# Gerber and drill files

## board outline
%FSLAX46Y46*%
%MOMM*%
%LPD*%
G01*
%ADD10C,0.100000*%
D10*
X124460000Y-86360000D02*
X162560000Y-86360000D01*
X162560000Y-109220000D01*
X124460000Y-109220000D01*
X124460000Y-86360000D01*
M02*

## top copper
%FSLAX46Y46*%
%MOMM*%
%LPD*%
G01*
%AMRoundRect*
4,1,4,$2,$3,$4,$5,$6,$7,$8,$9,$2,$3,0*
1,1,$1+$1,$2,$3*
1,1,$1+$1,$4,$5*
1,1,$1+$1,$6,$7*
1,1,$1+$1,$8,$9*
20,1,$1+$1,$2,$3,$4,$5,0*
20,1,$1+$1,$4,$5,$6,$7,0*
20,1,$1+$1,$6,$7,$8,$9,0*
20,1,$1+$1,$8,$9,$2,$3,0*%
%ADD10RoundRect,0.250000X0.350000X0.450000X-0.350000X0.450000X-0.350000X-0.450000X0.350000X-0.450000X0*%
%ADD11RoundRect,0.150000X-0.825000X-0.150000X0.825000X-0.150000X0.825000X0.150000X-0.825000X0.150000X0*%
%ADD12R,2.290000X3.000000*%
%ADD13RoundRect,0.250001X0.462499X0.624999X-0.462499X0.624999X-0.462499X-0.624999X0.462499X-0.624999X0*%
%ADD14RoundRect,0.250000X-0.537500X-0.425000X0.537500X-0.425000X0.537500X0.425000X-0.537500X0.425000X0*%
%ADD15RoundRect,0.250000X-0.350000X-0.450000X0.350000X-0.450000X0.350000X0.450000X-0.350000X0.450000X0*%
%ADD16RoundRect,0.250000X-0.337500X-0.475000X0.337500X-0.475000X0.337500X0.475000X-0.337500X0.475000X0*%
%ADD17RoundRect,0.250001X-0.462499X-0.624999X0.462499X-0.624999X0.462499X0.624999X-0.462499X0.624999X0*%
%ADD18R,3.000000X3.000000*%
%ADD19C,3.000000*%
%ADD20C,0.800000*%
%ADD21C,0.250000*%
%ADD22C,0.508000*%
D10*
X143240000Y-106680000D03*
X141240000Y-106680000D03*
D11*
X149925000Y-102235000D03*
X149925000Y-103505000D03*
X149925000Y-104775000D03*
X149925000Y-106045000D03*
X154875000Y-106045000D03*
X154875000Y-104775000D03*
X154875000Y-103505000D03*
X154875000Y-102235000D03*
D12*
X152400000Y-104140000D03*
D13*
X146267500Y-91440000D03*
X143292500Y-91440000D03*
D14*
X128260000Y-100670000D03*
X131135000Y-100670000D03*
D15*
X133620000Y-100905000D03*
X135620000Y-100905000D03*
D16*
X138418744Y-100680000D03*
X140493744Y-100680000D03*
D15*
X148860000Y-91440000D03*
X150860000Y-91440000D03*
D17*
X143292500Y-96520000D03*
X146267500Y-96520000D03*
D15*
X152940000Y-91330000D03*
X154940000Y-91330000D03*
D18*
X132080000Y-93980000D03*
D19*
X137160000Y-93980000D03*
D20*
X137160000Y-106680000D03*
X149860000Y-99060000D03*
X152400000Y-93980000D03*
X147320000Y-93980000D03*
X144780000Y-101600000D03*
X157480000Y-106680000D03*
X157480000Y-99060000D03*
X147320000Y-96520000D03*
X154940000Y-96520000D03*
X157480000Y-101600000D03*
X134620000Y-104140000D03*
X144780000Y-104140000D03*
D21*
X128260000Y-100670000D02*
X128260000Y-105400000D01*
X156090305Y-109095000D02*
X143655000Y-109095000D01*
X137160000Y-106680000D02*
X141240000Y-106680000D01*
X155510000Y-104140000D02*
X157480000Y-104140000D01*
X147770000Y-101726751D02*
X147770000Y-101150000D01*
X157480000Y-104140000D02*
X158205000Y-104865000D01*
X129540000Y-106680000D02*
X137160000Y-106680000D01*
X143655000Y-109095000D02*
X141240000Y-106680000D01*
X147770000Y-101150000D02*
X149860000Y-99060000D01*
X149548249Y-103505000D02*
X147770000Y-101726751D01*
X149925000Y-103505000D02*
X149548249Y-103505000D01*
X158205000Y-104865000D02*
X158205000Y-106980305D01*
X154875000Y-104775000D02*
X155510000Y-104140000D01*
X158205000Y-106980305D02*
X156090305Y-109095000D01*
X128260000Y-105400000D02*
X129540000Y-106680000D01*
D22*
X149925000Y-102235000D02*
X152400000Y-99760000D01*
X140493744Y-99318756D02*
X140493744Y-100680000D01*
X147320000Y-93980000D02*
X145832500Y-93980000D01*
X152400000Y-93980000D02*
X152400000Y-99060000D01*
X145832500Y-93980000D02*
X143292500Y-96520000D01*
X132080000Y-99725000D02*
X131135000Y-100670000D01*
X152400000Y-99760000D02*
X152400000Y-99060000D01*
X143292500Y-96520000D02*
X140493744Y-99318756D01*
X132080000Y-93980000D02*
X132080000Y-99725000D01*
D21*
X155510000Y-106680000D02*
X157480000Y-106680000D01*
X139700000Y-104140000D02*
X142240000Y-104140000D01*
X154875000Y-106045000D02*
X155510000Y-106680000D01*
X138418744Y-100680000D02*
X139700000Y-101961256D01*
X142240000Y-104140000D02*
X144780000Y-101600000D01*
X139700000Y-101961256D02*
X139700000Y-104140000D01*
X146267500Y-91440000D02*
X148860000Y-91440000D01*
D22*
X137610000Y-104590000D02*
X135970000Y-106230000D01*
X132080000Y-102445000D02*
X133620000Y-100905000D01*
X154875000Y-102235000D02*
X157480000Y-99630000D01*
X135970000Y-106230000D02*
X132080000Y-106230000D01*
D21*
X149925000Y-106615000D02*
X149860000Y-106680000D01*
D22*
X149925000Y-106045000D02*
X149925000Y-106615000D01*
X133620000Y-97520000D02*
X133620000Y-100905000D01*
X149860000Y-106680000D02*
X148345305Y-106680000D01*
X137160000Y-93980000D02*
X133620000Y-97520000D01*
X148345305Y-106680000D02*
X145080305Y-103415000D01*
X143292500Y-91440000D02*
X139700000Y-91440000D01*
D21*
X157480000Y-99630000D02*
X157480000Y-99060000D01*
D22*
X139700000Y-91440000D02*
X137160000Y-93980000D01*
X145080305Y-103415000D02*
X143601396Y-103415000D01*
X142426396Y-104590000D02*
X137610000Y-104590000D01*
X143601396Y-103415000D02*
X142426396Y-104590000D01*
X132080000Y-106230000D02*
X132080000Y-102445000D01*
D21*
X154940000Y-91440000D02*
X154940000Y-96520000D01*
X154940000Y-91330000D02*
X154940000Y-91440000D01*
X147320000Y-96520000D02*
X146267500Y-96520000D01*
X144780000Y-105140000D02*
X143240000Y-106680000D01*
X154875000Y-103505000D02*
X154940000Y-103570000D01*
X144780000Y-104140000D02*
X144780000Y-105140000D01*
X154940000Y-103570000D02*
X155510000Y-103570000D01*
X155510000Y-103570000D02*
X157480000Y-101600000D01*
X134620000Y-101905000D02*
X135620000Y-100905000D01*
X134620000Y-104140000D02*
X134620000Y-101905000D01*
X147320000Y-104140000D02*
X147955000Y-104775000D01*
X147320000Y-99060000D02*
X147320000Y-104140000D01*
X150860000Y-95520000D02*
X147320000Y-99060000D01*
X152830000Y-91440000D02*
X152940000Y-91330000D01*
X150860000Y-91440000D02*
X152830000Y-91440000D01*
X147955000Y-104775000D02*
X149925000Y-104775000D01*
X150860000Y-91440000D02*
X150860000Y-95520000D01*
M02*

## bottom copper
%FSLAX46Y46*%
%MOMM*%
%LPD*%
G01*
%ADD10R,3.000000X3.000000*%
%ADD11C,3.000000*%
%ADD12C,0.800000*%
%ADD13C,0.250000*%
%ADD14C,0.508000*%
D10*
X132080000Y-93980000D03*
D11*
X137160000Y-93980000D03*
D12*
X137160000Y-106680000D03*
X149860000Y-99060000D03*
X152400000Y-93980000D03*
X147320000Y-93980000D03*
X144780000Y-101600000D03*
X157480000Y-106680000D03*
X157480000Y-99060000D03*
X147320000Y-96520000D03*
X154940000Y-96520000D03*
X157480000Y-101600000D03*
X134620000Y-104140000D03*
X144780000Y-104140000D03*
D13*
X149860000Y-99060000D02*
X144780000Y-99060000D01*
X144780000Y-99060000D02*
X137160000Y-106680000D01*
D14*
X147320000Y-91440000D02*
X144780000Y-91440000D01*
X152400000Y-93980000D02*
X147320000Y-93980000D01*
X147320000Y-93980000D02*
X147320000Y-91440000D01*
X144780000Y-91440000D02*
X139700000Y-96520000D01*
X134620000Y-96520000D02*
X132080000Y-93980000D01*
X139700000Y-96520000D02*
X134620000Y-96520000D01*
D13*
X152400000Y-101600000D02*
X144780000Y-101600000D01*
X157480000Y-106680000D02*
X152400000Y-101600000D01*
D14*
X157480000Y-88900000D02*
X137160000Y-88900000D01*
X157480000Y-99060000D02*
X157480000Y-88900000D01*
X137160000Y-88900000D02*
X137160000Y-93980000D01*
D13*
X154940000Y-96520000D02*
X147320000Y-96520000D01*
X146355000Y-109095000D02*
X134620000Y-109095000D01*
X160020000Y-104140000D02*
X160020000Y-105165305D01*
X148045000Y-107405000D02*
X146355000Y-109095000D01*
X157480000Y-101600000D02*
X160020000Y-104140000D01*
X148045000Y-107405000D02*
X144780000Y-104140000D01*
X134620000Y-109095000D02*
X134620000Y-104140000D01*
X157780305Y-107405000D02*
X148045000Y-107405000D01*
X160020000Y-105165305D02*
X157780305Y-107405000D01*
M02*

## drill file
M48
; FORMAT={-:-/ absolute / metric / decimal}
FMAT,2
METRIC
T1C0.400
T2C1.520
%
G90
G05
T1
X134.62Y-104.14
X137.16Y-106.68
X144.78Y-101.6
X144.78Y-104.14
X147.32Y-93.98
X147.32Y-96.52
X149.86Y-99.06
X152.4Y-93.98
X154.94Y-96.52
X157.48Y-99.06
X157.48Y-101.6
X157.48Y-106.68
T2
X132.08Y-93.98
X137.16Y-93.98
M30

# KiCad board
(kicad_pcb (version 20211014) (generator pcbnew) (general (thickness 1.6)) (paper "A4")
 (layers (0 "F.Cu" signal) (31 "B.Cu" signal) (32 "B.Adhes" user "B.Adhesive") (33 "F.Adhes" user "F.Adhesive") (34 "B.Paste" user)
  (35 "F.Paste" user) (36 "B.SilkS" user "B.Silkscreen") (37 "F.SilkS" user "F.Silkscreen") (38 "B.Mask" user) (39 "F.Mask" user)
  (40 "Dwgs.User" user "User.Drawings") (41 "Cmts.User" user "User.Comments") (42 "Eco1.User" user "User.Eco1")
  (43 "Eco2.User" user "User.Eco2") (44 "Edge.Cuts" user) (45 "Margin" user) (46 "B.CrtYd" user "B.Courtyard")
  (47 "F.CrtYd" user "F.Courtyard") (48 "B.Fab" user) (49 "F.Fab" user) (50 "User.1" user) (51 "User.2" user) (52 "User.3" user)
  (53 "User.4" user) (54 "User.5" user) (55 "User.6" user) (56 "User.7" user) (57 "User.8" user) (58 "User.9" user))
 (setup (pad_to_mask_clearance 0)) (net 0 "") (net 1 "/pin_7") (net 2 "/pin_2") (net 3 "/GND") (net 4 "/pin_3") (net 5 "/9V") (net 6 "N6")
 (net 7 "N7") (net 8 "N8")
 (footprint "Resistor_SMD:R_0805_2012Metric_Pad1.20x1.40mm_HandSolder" (layer "F.Cu") (at 142.24 106.68 180)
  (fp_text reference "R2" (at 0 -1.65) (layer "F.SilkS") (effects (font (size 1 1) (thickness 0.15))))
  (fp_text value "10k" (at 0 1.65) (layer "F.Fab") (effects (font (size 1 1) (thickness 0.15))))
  (pad "1" smd roundrect (at -1 0 180) (size 1.2 1.4) (layers "F.Cu" "F.Paste" "F.Mask") (roundrect_rratio 0.208333) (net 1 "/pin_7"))
  (pad "2" smd roundrect (at 1 0 180) (size 1.2 1.4) (layers "F.Cu" "F.Paste" "F.Mask") (roundrect_rratio 0.208333) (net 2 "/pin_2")))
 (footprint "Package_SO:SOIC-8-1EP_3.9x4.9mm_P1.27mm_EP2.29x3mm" (layer "F.Cu") (at 152.4 104.14)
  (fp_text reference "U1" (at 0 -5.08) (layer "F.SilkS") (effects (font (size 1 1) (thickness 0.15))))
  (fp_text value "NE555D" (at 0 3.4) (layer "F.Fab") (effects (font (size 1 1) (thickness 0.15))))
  (pad "" smd roundrect (at 0.57 -0.75) (size 0.92 1.21) (layers "F.Paste") (roundrect_rratio 0.25))
  (pad "" smd roundrect (at -0.57 0.75) (size 0.92 1.21) (layers "F.Paste") (roundrect_rratio 0.25))
  (pad "" smd roundrect (at 0.57 0.75) (size 0.92 1.21) (layers "F.Paste") (roundrect_rratio 0.25))
  (pad "" smd roundrect (at -0.57 -0.75) (size 0.92 1.21) (layers "F.Paste") (roundrect_rratio 0.25))
  (pad "1" smd roundrect (at -2.475 -1.905) (size 1.95 0.6) (layers "F.Cu" "F.Paste" "F.Mask") (roundrect_rratio 0.25) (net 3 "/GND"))
  (pad "2" smd roundrect (at -2.475 -0.635) (size 1.95 0.6) (layers "F.Cu" "F.Paste" "F.Mask") (roundrect_rratio 0.25) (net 2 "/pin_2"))
  (pad "3" smd roundrect (at -2.475 0.635) (size 1.95 0.6) (layers "F.Cu" "F.Paste" "F.Mask") (roundrect_rratio 0.25) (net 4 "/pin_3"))
  (pad "4" smd roundrect (at -2.475 1.905) (size 1.95 0.6) (layers "F.Cu" "F.Paste" "F.Mask") (roundrect_rratio 0.25) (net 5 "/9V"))
  (pad "5" smd roundrect (at 2.475 1.905) (size 1.95 0.6) (layers "F.Cu" "F.Paste" "F.Mask") (roundrect_rratio 0.25) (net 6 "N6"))
  (pad "6" smd roundrect (at 2.475 0.635) (size 1.95 0.6) (layers "F.Cu" "F.Paste" "F.Mask") (roundrect_rratio 0.25) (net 2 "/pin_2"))
  (pad "7" smd roundrect (at 2.475 -0.635) (size 1.95 0.6) (layers "F.Cu" "F.Paste" "F.Mask") (roundrect_rratio 0.25) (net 1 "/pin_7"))
  (pad "8" smd roundrect (at 2.475 -1.905) (size 1.95 0.6) (layers "F.Cu" "F.Paste" "F.Mask") (roundrect_rratio 0.25) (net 5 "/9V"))
  (pad "9" smd rect (at 0 0) (size 2.29 3) (layers "F.Cu" "F.Mask")))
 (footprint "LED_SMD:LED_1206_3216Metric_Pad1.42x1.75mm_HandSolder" (layer "F.Cu") (at 144.78 91.44 180)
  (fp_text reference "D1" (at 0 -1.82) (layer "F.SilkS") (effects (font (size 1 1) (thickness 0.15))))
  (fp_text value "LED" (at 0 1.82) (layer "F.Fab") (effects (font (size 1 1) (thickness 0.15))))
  (pad "1" smd roundrect (at -1.4875 0 180) (size 1.425 1.75) (layers "F.Cu" "F.Paste" "F.Mask") (roundrect_rratio 0.175439) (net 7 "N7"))
  (pad "2" smd roundrect (at 1.4875 0 180) (size 1.425 1.75) (layers "F.Cu" "F.Paste" "F.Mask") (roundrect_rratio 0.175439) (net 5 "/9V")))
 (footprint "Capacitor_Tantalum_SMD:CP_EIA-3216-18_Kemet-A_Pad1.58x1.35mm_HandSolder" (layer "F.Cu") (at 129.6975 100.67)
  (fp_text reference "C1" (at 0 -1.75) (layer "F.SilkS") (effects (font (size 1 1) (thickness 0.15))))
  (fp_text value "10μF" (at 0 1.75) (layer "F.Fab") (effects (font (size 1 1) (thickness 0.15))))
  (pad "1" smd roundrect (at -1.4375 0) (size 1.575 1.35) (layers "F.Cu" "F.Paste" "F.Mask") (roundrect_rratio 0.185185) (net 2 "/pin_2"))
  (pad "2" smd roundrect (at 1.4375 0) (size 1.575 1.35) (layers "F.Cu" "F.Paste" "F.Mask") (roundrect_rratio 0.185185) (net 3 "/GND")))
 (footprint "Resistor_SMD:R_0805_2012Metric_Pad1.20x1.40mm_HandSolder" (layer "F.Cu") (at 134.62 100.905)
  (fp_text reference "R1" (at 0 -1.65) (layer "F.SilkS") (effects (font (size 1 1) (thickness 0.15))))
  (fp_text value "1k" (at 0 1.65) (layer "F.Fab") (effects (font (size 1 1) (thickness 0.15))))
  (pad "1" smd roundrect (at -1 0) (size 1.2 1.4) (layers "F.Cu" "F.Paste" "F.Mask") (roundrect_rratio 0.208333) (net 5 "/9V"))
  (pad "2" smd roundrect (at 1 0) (size 1.2 1.4) (layers "F.Cu" "F.Paste" "F.Mask") (roundrect_rratio 0.208333) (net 1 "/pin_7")))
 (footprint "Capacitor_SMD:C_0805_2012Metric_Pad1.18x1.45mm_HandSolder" (layer "F.Cu") (at 139.456244 100.68)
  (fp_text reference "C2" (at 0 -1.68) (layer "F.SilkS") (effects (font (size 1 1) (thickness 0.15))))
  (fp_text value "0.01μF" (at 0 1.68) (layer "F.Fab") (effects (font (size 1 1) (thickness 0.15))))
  (pad "1" smd roundrect (at -1.0375 0) (size 1.175 1.45) (layers "F.Cu" "F.Paste" "F.Mask") (roundrect_rratio 0.212766) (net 6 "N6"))
  (pad "2" smd roundrect (at 1.0375 0) (size 1.175 1.45) (layers "F.Cu" "F.Paste" "F.Mask") (roundrect_rratio 0.212766) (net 3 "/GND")))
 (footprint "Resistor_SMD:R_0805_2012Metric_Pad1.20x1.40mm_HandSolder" (layer "F.Cu") (at 149.86 91.44)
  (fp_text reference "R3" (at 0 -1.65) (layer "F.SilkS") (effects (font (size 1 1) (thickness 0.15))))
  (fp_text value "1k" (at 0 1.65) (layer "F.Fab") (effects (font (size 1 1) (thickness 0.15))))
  (pad "1" smd roundrect (at -1 0) (size 1.2 1.4) (layers "F.Cu" "F.Paste" "F.Mask") (roundrect_rratio 0.208333) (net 7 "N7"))
  (pad "2" smd roundrect (at 1 0) (size 1.2 1.4) (layers "F.Cu" "F.Paste" "F.Mask") (roundrect_rratio 0.208333) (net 4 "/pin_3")))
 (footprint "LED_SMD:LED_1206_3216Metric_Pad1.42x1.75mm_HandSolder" (layer "F.Cu") (at 144.78 96.52)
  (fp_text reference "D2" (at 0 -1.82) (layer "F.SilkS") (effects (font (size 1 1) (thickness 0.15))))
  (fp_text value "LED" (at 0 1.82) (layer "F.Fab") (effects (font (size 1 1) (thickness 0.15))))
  (pad "1" smd roundrect (at -1.4875 0) (size 1.425 1.75) (layers "F.Cu" "F.Paste" "F.Mask") (roundrect_rratio 0.175439) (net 3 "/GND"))
  (pad "2" smd roundrect (at 1.4875 0) (size 1.425 1.75) (layers "F.Cu" "F.Paste" "F.Mask") (roundrect_rratio 0.175439) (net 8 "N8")))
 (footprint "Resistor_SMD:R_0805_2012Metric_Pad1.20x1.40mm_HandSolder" (layer "F.Cu") (at 153.94 91.33)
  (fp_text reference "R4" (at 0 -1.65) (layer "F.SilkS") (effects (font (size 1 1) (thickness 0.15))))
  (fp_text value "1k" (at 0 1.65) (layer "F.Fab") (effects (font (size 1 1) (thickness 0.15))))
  (pad "1" smd roundrect (at -1 0) (size 1.2 1.4) (layers "F.Cu" "F.Paste" "F.Mask") (roundrect_rratio 0.208333) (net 4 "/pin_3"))
  (pad "2" smd roundrect (at 1 0) (size 1.2 1.4) (layers "F.Cu" "F.Paste" "F.Mask") (roundrect_rratio 0.208333) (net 8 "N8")))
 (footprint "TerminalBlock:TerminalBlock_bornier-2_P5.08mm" (layer "F.Cu") (at 132.08 93.98)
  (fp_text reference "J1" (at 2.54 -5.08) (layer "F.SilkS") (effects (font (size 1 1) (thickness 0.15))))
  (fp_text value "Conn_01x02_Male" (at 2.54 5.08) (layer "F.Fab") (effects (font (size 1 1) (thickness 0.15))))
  (pad "1" thru_hole rect (at 0 0) (size 3 3) (drill 1.52) (layers *.Cu *.Mask) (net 3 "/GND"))
  (pad "2" thru_hole circle (at 5.08 0) (size 3 3) (drill 1.52) (layers *.Cu *.Mask) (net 5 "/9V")))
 (gr_rect (start 124.46 86.36) (end 162.56 109.22) (layer "Edge.Cuts") (width 0.1) (fill none))
 (segment (start 128.26 100.67) (end 128.26 105.4) (width 0.25) (layer "F.Cu") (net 2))
 (segment (start 156.090305 109.095) (end 143.655 109.095) (width 0.25) (layer "F.Cu") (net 2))
 (segment (start 137.16 106.68) (end 141.24 106.68) (width 0.25) (layer "F.Cu") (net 2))
 (segment (start 155.51 104.14) (end 157.48 104.14) (width 0.25) (layer "F.Cu") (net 2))
 (segment (start 147.77 101.726751) (end 147.77 101.15) (width 0.25) (layer "F.Cu") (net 2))
 (segment (start 157.48 104.14) (end 158.205 104.865) (width 0.25) (layer "F.Cu") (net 2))
 (segment (start 129.54 106.68) (end 137.16 106.68) (width 0.25) (layer "F.Cu") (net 2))
 (segment (start 143.655 109.095) (end 141.24 106.68) (width 0.25) (layer "F.Cu") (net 2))
 (segment (start 147.77 101.15) (end 149.86 99.06) (width 0.25) (layer "F.Cu") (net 2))
 (segment (start 149.548249 103.505) (end 147.77 101.726751) (width 0.25) (layer "F.Cu") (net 2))
 (segment (start 149.925 103.505) (end 149.548249 103.505) (width 0.25) (layer "F.Cu") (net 2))
 (segment (start 158.205 104.865) (end 158.205 106.980305) (width 0.25) (layer "F.Cu") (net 2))
 (segment (start 154.875 104.775) (end 155.51 104.14) (width 0.25) (layer "F.Cu") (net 2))
 (segment (start 158.205 106.980305) (end 156.090305 109.095) (width 0.25) (layer "F.Cu") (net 2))
 (segment (start 128.26 105.4) (end 129.54 106.68) (width 0.25) (layer "F.Cu") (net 2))
 (via (at 137.16 106.68) (size 0.8) (drill 0.4) (layers "F.Cu" "B.Cu") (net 2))
 (via (at 149.86 99.06) (size 0.8) (drill 0.4) (layers "F.Cu" "B.Cu") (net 2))
 (segment (start 149.86 99.06) (end 144.78 99.06) (width 0.25) (layer "B.Cu") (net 2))
 (segment (start 144.78 99.06) (end 137.16 106.68) (width 0.25) (layer "B.Cu") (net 2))
 (segment (start 149.925 102.235) (end 152.4 99.76) (width 0.508) (layer "F.Cu") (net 3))
 (segment (start 140.493744 99.318756) (end 140.493744 100.68) (width 0.508) (layer "F.Cu") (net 3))
 (segment (start 147.32 93.98) (end 145.8325 93.98) (width 0.508) (layer "F.Cu") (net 3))
 (segment (start 152.4 93.98) (end 152.4 99.06) (width 0.508) (layer "F.Cu") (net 3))
 (segment (start 145.8325 93.98) (end 143.2925 96.52) (width 0.508) (layer "F.Cu") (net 3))
 (segment (start 132.08 99.725) (end 131.135 100.67) (width 0.508) (layer "F.Cu") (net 3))
 (segment (start 152.4 99.76) (end 152.4 99.06) (width 0.508) (layer "F.Cu") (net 3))
 (segment (start 143.2925 96.52) (end 140.493744 99.318756) (width 0.508) (layer "F.Cu") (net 3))
 (segment (start 132.08 93.98) (end 132.08 99.725) (width 0.508) (layer "F.Cu") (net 3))
 (via (at 152.4 93.98) (size 0.8) (drill 0.4) (layers "F.Cu" "B.Cu") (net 3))
 (via (at 147.32 93.98) (size 0.8) (drill 0.4) (layers "F.Cu" "B.Cu") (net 3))
 (segment (start 147.32 91.44) (end 144.78 91.44) (width 0.508) (layer "B.Cu") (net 3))
 (segment (start 152.4 93.98) (end 147.32 93.98) (width 0.508) (layer "B.Cu") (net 3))
 (segment (start 147.32 93.98) (end 147.32 91.44) (width 0.508) (layer "B.Cu") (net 3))
 (segment (start 144.78 91.44) (end 139.7 96.52) (width 0.508) (layer "B.Cu") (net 3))
 (segment (start 134.62 96.52) (end 132.08 93.98) (width 0.508) (layer "B.Cu") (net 3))
 (segment (start 139.7 96.52) (end 134.62 96.52) (width 0.508) (layer "B.Cu") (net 3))
 (segment (start 155.51 106.68) (end 157.48 106.68) (width 0.25) (layer "F.Cu") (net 6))
 (segment (start 139.7 104.14) (end 142.24 104.14) (width 0.25) (layer "F.Cu") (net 6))
 (segment (start 154.875 106.045) (end 155.51 106.68) (width 0.25) (layer "F.Cu") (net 6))
 (segment (start 138.418744 100.68) (end 139.7 101.961256) (width 0.25) (layer "F.Cu") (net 6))
 (segment (start 142.24 104.14) (end 144.78 101.6) (width 0.25) (layer "F.Cu") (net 6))
 (segment (start 139.7 101.961256) (end 139.7 104.14) (width 0.25) (layer "F.Cu") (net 6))
 (via (at 144.78 101.6) (size 0.8) (drill 0.4) (layers "F.Cu" "B.Cu") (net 6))
 (via (at 157.48 106.68) (size 0.8) (drill 0.4) (layers "F.Cu" "B.Cu") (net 6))
 (segment (start 152.4 101.6) (end 144.78 101.6) (width 0.25) (layer "B.Cu") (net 6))
 (segment (start 157.48 106.68) (end 152.4 101.6) (width 0.25) (layer "B.Cu") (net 6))
 (segment (start 146.2675 91.44) (end 148.86 91.44) (width 0.25) (layer "F.Cu") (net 7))
 (segment (start 137.61 104.59) (end 135.97 106.23) (width 0.508) (layer "F.Cu") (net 5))
 (segment (start 132.08 102.445) (end 133.62 100.905) (width 0.508) (layer "F.Cu") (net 5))
 (segment (start 154.875 102.235) (end 157.48 99.63) (width 0.508) (layer "F.Cu") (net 5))
 (segment (start 135.97 106.23) (end 132.08 106.23) (width 0.508) (layer "F.Cu") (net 5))
 (segment (start 149.925 106.615) (end 149.86 106.68) (width 0.25) (layer "F.Cu") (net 5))
 (segment (start 149.925 106.045) (end 149.925 106.615) (width 0.508) (layer "F.Cu") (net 5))
 (segment (start 133.62 97.52) (end 133.62 100.905) (width 0.508) (layer "F.Cu") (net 5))
 (segment (start 149.86 106.68) (end 148.345305 106.68) (width 0.508) (layer "F.Cu") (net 5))
 (segment (start 137.16 93.98) (end 133.62 97.52) (width 0.508) (layer "F.Cu") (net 5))
 (segment (start 148.345305 106.68) (end 145.080305 103.415) (width 0.508) (layer "F.Cu") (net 5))
 (segment (start 143.2925 91.44) (end 139.7 91.44) (width 0.508) (layer "F.Cu") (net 5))
 (segment (start 157.48 99.63) (end 157.48 99.06) (width 0.25) (layer "F.Cu") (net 5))
 (segment (start 139.7 91.44) (end 137.16 93.98) (width 0.508) (layer "F.Cu") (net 5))
 (segment (start 145.080305 103.415) (end 143.601396 103.415) (width 0.508) (layer "F.Cu") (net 5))
 (segment (start 142.426396 104.59) (end 137.61 104.59) (width 0.508) (layer "F.Cu") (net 5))
 (segment (start 143.601396 103.415) (end 142.426396 104.59) (width 0.508) (layer "F.Cu") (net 5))
 (segment (start 132.08 106.23) (end 132.08 102.445) (width 0.508) (layer "F.Cu") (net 5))
 (via (at 157.48 99.06) (size 0.8) (drill 0.4) (layers "F.Cu" "B.Cu") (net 5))
 (segment (start 157.48 88.9) (end 137.16 88.9) (width 0.508) (layer "B.Cu") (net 5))
 (segment (start 157.48 99.06) (end 157.48 88.9) (width 0.508) (layer "B.Cu") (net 5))
 (segment (start 137.16 88.9) (end 137.16 93.98) (width 0.508) (layer "B.Cu") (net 5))
 (segment (start 154.94 91.44) (end 154.94 96.52) (width 0.25) (layer "F.Cu") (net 8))
 (segment (start 154.94 91.33) (end 154.94 91.44) (width 0.25) (layer "F.Cu") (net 8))
 (segment (start 147.32 96.52) (end 146.2675 96.52) (width 0.25) (layer "F.Cu") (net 8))
 (via (at 147.32 96.52) (size 0.8) (drill 0.4) (layers "F.Cu" "B.Cu") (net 8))
 (via (at 154.94 96.52) (size 0.8) (drill 0.4) (layers "F.Cu" "B.Cu") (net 8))
 (segment (start 154.94 96.52) (end 147.32 96.52) (width 0.25) (layer "B.Cu") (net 8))
 (segment (start 144.78 105.14) (end 143.24 106.68) (width 0.25) (layer "F.Cu") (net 1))
 (segment (start 154.875 103.505) (end 154.94 103.57) (width 0.25) (layer "F.Cu") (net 1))
 (segment (start 144.78 104.14) (end 144.78 105.14) (width 0.25) (layer "F.Cu") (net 1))
 (segment (start 154.94 103.57) (end 155.51 103.57) (width 0.25) (layer "F.Cu") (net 1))
 (segment (start 155.51 103.57) (end 157.48 101.6) (width 0.25) (layer "F.Cu") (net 1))
 (segment (start 134.62 101.905) (end 135.62 100.905) (width 0.25) (layer "F.Cu") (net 1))
 (segment (start 134.62 104.14) (end 134.62 101.905) (width 0.25) (layer "F.Cu") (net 1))
 (via (at 157.48 101.6) (size 0.8) (drill 0.4) (layers "F.Cu" "B.Cu") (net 1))
 (via (at 134.62 104.14) (size 0.8) (drill 0.4) (layers "F.Cu" "B.Cu") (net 1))
 (via (at 144.78 104.14) (size 0.8) (drill 0.4) (layers "F.Cu" "B.Cu") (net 1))
 (segment (start 146.355 109.095) (end 134.62 109.095) (width 0.25) (layer "B.Cu") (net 1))
 (segment (start 160.02 104.14) (end 160.02 105.165305) (width 0.25) (layer "B.Cu") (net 1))
 (segment (start 148.045 107.405) (end 146.355 109.095) (width 0.25) (layer "B.Cu") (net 1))
 (segment (start 157.48 101.6) (end 160.02 104.14) (width 0.25) (layer "B.Cu") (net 1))
 (segment (start 148.045 107.405) (end 144.78 104.14) (width 0.25) (layer "B.Cu") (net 1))
 (segment (start 134.62 109.095) (end 134.62 104.14) (width 0.25) (layer "B.Cu") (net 1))
 (segment (start 157.780305 107.405) (end 148.045 107.405) (width 0.25) (layer "B.Cu") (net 1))
 (segment (start 160.02 105.165305) (end 157.780305 107.405) (width 0.25) (layer "B.Cu") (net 1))
 (segment (start 147.32 104.14) (end 147.955 104.775) (width 0.25) (layer "F.Cu") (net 4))
 (segment (start 147.32 99.06) (end 147.32 104.14) (width 0.25) (layer "F.Cu") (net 4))
 (segment (start 150.86 95.52) (end 147.32 99.06) (width 0.25) (layer "F.Cu") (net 4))
 (segment (start 152.83 91.44) (end 152.94 91.33) (width 0.25) (layer "F.Cu") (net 4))
 (segment (start 150.86 91.44) (end 152.83 91.44) (width 0.25) (layer "F.Cu") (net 4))
 (segment (start 147.955 104.775) (end 149.925 104.775) (width 0.25) (layer "F.Cu") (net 4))
 (segment (start 150.86 91.44) (end 150.86 95.52) (width 0.25) (layer "F.Cu") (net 4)))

